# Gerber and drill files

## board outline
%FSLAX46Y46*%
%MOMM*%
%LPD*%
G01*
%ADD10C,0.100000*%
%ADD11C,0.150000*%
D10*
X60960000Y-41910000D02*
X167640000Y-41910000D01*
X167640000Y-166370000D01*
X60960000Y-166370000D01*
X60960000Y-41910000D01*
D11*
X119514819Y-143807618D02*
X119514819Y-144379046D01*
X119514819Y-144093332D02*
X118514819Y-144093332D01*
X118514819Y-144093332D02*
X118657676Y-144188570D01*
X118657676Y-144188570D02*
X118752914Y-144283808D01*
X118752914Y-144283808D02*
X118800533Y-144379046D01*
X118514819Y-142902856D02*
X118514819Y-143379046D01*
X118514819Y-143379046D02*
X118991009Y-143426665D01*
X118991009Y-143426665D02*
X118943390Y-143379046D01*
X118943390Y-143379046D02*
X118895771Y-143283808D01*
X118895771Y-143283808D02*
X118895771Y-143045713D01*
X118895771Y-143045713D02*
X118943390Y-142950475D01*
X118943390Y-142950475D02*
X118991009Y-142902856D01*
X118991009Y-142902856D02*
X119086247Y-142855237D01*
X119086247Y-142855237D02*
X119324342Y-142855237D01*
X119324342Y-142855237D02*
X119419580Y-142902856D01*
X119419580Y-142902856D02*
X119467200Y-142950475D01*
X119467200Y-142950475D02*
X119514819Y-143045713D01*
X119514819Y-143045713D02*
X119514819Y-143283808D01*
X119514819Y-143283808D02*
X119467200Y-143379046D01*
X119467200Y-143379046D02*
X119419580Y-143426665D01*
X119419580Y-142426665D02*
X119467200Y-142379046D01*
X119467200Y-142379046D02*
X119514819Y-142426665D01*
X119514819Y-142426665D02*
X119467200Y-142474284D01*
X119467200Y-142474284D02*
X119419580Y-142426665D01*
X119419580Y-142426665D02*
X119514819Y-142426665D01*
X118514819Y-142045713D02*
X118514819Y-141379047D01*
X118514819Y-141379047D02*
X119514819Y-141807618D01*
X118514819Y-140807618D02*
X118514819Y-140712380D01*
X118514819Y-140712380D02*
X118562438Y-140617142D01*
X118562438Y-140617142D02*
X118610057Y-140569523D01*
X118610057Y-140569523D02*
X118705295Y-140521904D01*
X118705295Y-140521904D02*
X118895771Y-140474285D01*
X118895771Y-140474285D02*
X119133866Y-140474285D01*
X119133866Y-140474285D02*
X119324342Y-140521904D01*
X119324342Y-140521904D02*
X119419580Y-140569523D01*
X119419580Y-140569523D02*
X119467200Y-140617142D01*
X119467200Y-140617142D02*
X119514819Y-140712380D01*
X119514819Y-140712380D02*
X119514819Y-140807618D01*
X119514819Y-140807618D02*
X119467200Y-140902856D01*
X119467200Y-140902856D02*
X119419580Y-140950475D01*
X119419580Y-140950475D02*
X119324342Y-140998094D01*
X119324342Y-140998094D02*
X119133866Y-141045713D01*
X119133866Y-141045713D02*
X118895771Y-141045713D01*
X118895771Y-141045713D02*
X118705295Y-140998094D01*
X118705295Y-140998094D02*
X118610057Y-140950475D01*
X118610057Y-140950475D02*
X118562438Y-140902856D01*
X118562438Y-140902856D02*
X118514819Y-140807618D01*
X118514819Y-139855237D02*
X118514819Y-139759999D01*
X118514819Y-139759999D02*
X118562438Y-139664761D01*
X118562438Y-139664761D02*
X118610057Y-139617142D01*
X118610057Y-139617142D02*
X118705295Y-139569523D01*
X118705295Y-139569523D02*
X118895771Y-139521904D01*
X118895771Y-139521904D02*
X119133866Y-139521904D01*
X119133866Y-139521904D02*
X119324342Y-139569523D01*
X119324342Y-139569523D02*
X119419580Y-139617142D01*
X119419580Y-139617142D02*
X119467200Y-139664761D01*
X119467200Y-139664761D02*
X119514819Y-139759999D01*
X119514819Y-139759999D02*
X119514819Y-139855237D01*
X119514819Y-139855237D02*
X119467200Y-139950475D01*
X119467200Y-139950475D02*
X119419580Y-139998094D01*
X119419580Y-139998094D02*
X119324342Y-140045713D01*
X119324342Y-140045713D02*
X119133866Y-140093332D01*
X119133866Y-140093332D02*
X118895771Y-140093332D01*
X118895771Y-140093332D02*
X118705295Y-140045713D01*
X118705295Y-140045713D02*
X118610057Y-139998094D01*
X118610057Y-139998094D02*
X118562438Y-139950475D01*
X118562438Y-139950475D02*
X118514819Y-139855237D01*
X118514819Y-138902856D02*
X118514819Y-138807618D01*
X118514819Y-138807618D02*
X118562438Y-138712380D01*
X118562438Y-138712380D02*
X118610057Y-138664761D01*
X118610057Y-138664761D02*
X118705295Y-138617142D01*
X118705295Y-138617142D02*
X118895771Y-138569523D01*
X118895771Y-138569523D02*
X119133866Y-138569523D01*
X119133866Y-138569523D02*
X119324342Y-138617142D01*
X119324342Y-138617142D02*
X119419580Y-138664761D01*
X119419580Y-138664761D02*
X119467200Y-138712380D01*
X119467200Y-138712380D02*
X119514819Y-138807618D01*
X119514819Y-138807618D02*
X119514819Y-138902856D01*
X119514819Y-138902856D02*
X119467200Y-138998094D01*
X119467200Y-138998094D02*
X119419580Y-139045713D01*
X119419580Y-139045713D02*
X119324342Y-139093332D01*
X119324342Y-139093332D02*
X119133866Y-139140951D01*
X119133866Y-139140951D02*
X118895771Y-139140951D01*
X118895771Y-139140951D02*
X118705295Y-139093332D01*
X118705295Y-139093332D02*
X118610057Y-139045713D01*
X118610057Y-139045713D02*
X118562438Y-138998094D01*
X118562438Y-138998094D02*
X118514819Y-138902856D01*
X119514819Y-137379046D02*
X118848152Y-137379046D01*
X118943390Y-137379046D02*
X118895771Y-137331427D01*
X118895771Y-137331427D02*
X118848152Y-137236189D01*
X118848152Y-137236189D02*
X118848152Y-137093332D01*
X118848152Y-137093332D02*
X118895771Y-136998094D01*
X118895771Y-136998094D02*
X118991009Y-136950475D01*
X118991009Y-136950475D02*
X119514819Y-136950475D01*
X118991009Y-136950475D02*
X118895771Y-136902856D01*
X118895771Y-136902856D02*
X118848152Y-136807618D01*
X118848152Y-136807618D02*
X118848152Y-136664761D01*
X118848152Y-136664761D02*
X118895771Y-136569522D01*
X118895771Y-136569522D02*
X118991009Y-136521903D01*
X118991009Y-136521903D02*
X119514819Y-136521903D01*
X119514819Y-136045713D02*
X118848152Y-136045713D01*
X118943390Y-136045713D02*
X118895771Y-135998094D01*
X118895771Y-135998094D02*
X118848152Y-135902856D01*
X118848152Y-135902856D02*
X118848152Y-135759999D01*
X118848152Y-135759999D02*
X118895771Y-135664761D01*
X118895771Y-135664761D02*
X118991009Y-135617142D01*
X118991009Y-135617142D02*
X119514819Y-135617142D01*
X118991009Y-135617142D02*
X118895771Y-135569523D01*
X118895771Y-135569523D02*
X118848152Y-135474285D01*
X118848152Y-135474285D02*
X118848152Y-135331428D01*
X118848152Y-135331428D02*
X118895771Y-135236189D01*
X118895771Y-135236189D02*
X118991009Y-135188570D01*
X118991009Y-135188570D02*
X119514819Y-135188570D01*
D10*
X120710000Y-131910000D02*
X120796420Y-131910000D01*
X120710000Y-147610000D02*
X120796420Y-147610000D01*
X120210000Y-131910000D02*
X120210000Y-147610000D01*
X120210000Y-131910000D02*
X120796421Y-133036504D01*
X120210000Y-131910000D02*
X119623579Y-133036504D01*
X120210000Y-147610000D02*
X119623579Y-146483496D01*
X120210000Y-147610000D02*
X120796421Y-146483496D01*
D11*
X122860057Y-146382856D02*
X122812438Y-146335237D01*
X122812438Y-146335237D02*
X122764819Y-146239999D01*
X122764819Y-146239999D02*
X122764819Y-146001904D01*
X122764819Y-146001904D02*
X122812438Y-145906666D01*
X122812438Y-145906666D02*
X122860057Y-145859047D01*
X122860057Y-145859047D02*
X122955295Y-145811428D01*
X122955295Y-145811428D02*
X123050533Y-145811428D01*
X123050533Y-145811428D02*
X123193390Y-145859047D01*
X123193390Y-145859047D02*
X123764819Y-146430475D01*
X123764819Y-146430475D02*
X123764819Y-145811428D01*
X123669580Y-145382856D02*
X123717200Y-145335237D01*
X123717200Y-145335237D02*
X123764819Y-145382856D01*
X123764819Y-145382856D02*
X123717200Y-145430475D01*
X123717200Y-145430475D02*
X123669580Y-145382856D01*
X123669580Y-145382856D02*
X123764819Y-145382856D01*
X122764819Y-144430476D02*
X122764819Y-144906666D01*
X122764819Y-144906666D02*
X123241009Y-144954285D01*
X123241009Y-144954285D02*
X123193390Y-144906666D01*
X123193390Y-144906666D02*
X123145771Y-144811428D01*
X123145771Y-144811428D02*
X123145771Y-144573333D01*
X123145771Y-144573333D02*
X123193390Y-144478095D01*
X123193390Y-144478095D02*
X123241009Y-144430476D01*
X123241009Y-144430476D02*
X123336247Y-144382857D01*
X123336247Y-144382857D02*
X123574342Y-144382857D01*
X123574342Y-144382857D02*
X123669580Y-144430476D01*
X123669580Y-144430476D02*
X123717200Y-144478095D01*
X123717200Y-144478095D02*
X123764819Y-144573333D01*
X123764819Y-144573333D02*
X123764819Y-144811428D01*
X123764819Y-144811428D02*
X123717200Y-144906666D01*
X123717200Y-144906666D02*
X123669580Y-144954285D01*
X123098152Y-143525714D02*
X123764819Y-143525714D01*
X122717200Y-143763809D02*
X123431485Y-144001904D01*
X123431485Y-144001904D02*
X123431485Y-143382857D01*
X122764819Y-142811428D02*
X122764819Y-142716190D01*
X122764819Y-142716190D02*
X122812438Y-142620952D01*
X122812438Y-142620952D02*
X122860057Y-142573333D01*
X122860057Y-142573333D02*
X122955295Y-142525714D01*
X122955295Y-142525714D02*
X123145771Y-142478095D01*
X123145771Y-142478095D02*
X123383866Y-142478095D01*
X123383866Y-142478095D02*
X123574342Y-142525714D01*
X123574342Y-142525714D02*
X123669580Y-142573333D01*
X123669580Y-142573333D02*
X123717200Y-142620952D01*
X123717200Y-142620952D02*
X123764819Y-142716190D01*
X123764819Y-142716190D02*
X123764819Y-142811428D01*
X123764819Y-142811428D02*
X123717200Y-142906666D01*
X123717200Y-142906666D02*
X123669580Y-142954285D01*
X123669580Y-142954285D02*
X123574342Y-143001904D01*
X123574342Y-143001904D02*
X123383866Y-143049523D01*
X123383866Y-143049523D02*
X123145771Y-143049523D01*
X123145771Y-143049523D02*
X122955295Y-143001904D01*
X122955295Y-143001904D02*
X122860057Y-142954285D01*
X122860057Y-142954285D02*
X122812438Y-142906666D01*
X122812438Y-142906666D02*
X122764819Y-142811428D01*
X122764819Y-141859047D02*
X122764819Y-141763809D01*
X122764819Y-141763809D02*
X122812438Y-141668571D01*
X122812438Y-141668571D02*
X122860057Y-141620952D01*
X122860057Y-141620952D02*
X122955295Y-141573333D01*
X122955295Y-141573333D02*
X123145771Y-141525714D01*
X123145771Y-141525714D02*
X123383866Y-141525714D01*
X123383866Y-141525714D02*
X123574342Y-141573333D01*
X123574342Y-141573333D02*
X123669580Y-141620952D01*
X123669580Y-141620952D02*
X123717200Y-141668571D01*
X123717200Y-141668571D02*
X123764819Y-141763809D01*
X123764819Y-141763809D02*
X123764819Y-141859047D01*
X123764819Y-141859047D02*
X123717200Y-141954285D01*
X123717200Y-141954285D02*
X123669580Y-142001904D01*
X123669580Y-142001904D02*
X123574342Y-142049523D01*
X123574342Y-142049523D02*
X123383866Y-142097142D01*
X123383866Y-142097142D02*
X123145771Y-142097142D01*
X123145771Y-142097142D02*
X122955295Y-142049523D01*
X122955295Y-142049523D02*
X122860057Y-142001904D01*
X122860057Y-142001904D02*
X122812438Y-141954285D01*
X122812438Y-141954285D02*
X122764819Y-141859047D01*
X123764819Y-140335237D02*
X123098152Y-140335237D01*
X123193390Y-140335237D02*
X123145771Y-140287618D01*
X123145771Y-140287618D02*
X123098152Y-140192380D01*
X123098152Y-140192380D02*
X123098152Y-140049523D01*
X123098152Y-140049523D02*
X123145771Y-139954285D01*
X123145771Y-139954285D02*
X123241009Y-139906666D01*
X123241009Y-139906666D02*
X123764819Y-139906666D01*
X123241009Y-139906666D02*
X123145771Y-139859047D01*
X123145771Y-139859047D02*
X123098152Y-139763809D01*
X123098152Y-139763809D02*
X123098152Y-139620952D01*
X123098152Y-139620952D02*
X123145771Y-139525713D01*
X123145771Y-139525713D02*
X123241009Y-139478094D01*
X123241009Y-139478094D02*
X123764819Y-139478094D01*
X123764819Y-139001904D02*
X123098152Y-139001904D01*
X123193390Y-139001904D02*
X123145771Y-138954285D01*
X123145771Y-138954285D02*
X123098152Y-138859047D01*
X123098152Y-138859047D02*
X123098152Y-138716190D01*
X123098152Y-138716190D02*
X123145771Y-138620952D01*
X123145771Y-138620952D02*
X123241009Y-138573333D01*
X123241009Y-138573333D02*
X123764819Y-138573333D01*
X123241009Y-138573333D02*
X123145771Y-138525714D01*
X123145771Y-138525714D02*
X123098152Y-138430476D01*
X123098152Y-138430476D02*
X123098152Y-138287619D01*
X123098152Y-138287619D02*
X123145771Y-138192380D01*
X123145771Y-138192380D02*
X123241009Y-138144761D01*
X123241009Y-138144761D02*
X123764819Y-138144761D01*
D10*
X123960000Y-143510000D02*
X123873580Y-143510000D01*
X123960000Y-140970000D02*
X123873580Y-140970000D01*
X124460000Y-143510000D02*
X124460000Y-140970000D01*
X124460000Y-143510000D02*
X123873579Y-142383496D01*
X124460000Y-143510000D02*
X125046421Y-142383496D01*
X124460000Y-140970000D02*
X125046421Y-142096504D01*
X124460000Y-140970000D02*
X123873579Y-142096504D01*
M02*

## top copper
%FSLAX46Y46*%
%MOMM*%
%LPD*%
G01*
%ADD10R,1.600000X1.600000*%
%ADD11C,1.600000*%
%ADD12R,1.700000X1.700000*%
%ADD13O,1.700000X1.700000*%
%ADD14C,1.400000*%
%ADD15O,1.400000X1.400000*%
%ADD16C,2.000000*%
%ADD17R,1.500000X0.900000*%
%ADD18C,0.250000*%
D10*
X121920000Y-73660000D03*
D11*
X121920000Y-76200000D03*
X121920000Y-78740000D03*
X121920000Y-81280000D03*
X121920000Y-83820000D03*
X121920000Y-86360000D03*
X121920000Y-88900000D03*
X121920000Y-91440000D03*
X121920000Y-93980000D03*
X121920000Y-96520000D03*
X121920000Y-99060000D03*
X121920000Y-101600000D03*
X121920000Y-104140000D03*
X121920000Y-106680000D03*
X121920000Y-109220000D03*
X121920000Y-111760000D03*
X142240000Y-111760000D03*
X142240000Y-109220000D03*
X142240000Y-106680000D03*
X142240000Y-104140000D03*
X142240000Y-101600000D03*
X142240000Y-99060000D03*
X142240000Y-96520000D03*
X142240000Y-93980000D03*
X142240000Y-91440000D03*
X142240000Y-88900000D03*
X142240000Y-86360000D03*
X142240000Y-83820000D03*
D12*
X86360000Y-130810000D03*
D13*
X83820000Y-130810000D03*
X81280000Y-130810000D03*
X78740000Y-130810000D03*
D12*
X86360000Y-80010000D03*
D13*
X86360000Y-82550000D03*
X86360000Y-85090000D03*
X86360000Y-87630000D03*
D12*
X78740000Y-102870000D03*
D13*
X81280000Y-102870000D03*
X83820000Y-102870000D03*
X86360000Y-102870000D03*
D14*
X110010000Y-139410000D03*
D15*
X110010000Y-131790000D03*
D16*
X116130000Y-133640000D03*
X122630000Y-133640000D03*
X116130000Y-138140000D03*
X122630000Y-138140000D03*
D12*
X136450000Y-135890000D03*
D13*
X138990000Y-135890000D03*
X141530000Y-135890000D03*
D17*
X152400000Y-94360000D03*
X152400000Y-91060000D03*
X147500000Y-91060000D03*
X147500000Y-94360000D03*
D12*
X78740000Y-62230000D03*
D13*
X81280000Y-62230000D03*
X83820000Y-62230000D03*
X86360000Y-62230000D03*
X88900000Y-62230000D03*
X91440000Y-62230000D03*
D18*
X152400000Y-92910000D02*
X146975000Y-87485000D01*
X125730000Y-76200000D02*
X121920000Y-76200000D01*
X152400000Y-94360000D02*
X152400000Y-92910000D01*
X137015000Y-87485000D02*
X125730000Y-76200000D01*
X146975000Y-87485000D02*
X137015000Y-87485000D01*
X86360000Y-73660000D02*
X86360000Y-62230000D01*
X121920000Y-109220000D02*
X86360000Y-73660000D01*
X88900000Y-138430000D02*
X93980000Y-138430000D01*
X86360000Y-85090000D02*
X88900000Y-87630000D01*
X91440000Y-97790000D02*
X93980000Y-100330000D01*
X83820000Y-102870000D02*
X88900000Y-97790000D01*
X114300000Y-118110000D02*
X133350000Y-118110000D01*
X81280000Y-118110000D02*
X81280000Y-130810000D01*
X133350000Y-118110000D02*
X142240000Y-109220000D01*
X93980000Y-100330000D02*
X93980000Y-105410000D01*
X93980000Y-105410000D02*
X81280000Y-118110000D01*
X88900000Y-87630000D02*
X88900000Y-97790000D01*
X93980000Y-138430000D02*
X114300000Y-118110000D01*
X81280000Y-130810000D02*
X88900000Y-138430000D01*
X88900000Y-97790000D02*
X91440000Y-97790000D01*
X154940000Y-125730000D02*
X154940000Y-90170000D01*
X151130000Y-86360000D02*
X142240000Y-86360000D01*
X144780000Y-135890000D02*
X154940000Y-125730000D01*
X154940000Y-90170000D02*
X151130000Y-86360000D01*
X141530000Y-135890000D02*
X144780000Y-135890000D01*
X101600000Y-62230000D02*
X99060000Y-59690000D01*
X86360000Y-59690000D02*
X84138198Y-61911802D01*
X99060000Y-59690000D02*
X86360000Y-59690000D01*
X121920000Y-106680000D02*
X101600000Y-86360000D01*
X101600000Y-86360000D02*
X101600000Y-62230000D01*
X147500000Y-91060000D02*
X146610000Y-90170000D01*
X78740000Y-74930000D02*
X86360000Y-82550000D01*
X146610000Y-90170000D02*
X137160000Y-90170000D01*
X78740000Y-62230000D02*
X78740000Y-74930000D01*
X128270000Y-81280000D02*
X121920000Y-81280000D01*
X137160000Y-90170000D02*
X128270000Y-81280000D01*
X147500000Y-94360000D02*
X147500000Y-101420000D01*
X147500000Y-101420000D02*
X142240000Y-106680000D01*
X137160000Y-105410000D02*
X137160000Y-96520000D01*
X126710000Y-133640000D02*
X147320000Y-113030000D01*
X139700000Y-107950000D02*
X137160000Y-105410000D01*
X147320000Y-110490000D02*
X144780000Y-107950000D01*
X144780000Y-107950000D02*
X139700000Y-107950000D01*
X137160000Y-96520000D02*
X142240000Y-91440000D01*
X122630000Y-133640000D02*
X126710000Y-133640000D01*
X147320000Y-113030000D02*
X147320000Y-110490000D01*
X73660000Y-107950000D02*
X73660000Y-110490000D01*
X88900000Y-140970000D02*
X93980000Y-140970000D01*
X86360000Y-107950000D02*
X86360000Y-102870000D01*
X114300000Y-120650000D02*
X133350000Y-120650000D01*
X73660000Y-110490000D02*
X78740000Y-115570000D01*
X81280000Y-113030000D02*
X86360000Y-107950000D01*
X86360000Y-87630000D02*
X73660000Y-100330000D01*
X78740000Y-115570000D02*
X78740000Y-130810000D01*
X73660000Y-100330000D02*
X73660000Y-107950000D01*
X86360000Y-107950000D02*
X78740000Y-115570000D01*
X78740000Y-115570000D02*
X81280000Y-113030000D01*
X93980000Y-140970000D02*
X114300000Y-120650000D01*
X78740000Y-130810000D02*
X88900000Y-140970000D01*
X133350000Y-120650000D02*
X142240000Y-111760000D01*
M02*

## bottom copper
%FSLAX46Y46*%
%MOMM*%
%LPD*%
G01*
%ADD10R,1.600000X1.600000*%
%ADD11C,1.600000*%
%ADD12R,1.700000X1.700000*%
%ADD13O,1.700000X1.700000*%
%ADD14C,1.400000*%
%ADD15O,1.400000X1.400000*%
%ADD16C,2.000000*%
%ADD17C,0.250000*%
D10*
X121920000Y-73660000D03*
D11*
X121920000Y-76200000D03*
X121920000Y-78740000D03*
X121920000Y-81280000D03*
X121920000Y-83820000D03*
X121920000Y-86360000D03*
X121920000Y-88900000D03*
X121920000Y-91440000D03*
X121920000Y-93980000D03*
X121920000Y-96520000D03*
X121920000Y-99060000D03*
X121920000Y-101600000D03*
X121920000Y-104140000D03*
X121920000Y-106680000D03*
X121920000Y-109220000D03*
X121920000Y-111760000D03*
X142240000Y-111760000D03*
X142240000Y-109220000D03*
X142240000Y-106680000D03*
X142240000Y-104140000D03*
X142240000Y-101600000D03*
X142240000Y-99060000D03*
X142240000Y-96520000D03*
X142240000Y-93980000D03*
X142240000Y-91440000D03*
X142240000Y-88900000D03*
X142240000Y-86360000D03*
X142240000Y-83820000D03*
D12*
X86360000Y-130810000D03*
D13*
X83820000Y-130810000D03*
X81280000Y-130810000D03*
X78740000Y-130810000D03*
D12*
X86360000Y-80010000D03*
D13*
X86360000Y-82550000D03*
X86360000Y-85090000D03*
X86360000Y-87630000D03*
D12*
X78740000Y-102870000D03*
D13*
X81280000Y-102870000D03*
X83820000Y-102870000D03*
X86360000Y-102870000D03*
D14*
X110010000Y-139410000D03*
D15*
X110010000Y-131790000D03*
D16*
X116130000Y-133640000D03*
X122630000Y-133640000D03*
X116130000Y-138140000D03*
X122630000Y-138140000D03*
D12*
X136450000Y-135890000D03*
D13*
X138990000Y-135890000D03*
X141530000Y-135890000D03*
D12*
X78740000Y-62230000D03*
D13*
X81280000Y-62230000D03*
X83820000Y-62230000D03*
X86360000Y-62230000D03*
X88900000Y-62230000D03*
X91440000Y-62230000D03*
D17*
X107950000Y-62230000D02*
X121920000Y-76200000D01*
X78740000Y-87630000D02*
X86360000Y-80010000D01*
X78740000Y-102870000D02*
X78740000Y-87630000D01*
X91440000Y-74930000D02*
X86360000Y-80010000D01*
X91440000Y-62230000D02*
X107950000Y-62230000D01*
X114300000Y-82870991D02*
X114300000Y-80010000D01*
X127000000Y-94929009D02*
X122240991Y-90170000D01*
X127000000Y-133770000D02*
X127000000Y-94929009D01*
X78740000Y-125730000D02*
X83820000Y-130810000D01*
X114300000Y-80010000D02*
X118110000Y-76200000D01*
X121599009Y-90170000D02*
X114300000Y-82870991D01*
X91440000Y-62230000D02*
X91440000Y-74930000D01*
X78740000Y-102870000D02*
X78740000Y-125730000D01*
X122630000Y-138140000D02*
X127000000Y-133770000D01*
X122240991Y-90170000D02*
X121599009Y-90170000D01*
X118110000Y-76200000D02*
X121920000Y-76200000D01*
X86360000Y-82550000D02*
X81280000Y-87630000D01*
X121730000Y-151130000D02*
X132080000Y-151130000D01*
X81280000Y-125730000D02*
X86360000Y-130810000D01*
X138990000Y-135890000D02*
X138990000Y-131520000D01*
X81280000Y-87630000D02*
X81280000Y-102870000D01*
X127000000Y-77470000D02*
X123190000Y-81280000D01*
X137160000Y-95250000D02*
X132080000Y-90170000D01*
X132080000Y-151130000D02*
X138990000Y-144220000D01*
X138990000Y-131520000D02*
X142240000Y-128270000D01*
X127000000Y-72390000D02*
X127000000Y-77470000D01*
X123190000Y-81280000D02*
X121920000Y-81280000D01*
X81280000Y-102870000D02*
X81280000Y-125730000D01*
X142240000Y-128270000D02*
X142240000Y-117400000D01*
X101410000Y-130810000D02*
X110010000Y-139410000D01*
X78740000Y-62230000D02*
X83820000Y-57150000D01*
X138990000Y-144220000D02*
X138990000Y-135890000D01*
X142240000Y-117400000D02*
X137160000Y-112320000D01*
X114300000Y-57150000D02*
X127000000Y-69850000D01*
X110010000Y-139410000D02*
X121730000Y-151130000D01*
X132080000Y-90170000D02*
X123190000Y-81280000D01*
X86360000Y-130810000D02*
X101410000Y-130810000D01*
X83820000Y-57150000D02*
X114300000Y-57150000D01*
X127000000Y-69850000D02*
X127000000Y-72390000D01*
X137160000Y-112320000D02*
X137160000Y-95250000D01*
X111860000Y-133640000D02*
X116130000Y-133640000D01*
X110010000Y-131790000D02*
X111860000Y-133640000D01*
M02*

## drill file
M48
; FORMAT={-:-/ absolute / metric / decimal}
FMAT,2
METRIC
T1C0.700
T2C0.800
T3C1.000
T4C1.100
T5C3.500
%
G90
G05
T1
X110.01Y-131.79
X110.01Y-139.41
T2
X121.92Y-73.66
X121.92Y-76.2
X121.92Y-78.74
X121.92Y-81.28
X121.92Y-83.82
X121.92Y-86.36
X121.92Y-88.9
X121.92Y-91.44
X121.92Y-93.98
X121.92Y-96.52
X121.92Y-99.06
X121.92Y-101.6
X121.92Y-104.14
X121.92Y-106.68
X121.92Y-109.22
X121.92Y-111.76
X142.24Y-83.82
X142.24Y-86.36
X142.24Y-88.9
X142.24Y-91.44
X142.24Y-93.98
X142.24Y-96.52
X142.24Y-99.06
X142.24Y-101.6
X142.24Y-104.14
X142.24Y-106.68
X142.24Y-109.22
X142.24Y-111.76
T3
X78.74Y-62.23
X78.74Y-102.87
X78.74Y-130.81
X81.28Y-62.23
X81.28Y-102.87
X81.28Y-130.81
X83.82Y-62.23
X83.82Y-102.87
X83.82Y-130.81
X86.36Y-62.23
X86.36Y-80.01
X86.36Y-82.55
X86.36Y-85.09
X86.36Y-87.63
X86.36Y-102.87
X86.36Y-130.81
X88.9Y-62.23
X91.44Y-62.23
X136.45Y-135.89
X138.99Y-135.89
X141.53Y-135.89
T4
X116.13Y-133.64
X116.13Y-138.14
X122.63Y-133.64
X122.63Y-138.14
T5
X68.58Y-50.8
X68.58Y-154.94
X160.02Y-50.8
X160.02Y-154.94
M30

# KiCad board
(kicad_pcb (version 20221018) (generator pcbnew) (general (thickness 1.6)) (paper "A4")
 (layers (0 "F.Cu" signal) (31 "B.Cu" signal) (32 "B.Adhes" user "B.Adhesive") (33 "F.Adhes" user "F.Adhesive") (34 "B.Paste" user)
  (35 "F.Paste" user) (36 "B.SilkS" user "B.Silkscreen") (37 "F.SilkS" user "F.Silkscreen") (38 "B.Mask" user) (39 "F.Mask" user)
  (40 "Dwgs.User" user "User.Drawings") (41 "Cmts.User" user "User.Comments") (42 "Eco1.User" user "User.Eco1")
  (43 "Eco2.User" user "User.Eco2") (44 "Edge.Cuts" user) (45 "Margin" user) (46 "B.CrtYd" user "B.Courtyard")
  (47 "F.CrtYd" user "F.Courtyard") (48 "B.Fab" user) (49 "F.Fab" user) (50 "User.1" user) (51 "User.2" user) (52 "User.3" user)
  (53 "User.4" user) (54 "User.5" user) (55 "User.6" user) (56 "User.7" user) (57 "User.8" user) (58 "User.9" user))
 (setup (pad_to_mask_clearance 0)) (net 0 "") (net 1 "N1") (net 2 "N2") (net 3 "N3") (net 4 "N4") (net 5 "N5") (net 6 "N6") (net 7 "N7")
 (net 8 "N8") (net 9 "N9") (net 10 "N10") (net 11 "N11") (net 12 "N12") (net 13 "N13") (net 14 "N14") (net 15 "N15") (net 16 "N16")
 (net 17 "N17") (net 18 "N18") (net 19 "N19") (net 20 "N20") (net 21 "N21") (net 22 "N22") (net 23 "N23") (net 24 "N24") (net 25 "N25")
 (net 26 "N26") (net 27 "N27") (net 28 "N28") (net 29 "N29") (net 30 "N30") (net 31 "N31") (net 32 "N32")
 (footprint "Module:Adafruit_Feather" (layer "F.Cu") (at 121.92 73.66)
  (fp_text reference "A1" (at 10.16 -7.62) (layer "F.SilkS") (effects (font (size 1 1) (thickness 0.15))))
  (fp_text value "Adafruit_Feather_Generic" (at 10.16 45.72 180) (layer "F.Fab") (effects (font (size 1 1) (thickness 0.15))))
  (pad "1" thru_hole rect (at 0 0 180) (size 1.6 1.6) (drill 0.8) (layers "*.Cu" "*.Mask") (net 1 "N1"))
  (pad "2" thru_hole circle (at 0 2.54 180) (size 1.6 1.6) (drill 0.8) (layers "*.Cu" "*.Mask") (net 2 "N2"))
  (pad "3" thru_hole circle (at 0 5.08 180) (size 1.6 1.6) (drill 0.8) (layers "*.Cu" "*.Mask") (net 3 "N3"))
  (pad "4" thru_hole circle (at 0 7.62 180) (size 1.6 1.6) (drill 0.8) (layers "*.Cu" "*.Mask") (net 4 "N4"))
  (pad "5" thru_hole circle (at 0 10.16 180) (size 1.6 1.6) (drill 0.8) (layers "*.Cu" "*.Mask") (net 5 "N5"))
  (pad "6" thru_hole circle (at 0 12.7 180) (size 1.6 1.6) (drill 0.8) (layers "*.Cu" "*.Mask") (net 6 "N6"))
  (pad "7" thru_hole circle (at 0 15.24 180) (size 1.6 1.6) (drill 0.8) (layers "*.Cu" "*.Mask") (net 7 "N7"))
  (pad "8" thru_hole circle (at 0 17.78 180) (size 1.6 1.6) (drill 0.8) (layers "*.Cu" "*.Mask") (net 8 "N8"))
  (pad "9" thru_hole circle (at 0 20.32 180) (size 1.6 1.6) (drill 0.8) (layers "*.Cu" "*.Mask") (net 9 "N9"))
  (pad "10" thru_hole circle (at 0 22.86 180) (size 1.6 1.6) (drill 0.8) (layers "*.Cu" "*.Mask") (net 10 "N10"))
  (pad "11" thru_hole circle (at 0 25.4 180) (size 1.6 1.6) (drill 0.8) (layers "*.Cu" "*.Mask") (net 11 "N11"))
  (pad "12" thru_hole circle (at 0 27.94 180) (size 1.6 1.6) (drill 0.8) (layers "*.Cu" "*.Mask") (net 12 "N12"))
  (pad "13" thru_hole circle (at 0 30.48 180) (size 1.6 1.6) (drill 0.8) (layers "*.Cu" "*.Mask") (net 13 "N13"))
  (pad "14" thru_hole circle (at 0 33.02 180) (size 1.6 1.6) (drill 0.8) (layers "*.Cu" "*.Mask") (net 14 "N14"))
  (pad "15" thru_hole circle (at 0 35.56 180) (size 1.6 1.6) (drill 0.8) (layers "*.Cu" "*.Mask") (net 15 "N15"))
  (pad "16" thru_hole circle (at 0 38.1 180) (size 1.6 1.6) (drill 0.8) (layers "*.Cu" "*.Mask") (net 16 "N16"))
  (pad "17" thru_hole circle (at 20.32 38.1 180) (size 1.6 1.6) (drill 0.8) (layers "*.Cu" "*.Mask") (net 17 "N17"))
  (pad "18" thru_hole circle (at 20.32 35.56 180) (size 1.6 1.6) (drill 0.8) (layers "*.Cu" "*.Mask") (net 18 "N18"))
  (pad "19" thru_hole circle (at 20.32 33.02 180) (size 1.6 1.6) (drill 0.8) (layers "*.Cu" "*.Mask") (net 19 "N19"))
  (pad "20" thru_hole circle (at 20.32 30.48 180) (size 1.6 1.6) (drill 0.8) (layers "*.Cu" "*.Mask") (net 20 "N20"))
  (pad "21" thru_hole circle (at 20.32 27.94 180) (size 1.6 1.6) (drill 0.8) (layers "*.Cu" "*.Mask") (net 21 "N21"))
  (pad "22" thru_hole circle (at 20.32 25.4 180) (size 1.6 1.6) (drill 0.8) (layers "*.Cu" "*.Mask") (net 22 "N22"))
  (pad "23" thru_hole circle (at 20.32 22.86 180) (size 1.6 1.6) (drill 0.8) (layers "*.Cu" "*.Mask") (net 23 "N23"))
  (pad "24" thru_hole circle (at 20.32 20.32 180) (size 1.6 1.6) (drill 0.8) (layers "*.Cu" "*.Mask") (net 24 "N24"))
  (pad "25" thru_hole circle (at 20.32 17.78 180) (size 1.6 1.6) (drill 0.8) (layers "*.Cu" "*.Mask") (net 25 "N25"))
  (pad "26" thru_hole circle (at 20.32 15.24 180) (size 1.6 1.6) (drill 0.8) (layers "*.Cu" "*.Mask") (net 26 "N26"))
  (pad "27" thru_hole circle (at 20.32 12.7 180) (size 1.6 1.6) (drill 0.8) (layers "*.Cu" "*.Mask") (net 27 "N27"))
  (pad "28" thru_hole circle (at 20.32 10.16 180) (size 1.6 1.6) (drill 0.8) (layers "*.Cu" "*.Mask") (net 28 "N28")))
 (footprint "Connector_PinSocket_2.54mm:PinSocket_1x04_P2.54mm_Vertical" (layer "F.Cu") (at 86.36 130.81 -90)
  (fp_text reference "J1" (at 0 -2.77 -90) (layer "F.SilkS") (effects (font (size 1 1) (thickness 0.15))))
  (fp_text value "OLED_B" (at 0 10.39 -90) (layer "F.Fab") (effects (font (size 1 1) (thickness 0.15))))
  (pad "1" thru_hole rect (at 0 0 270) (size 1.7 1.7) (drill 1) (layers "*.Cu" "*.Mask") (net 4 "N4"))
  (pad "2" thru_hole oval (at 0 2.54 270) (size 1.7 1.7) (drill 1) (layers "*.Cu" "*.Mask") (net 2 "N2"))
  (pad "3" thru_hole oval (at 0 5.08 270) (size 1.7 1.7) (drill 1) (layers "*.Cu" "*.Mask") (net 18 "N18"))
  (pad "4" thru_hole oval (at 0 7.62 270) (size 1.7 1.7) (drill 1) (layers "*.Cu" "*.Mask") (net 17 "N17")))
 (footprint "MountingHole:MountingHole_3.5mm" (layer "F.Cu") (at 68.58 154.94)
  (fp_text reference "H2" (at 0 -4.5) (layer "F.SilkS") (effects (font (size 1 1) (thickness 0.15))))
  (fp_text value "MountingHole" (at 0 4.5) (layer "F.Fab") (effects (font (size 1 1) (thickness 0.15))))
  (pad "" np_thru_hole circle (at 0 0) (size 3.5 3.5) (drill 3.5) (layers "*.Cu" "*.Mask")))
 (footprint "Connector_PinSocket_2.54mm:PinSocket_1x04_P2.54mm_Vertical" (layer "F.Cu") (at 86.36 80.01)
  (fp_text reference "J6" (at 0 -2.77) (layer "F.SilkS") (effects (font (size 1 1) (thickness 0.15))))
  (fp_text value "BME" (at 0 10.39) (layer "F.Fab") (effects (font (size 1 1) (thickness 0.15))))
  (pad "1" thru_hole rect (at 0 0) (size 1.7 1.7) (drill 1) (layers "*.Cu" "*.Mask") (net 2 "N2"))
  (pad "2" thru_hole oval (at 0 2.54) (size 1.7 1.7) (drill 1) (layers "*.Cu" "*.Mask") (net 4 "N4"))
  (pad "3" thru_hole oval (at 0 5.08) (size 1.7 1.7) (drill 1) (layers "*.Cu" "*.Mask") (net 18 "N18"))
  (pad "4" thru_hole oval (at 0 7.62) (size 1.7 1.7) (drill 1) (layers "*.Cu" "*.Mask") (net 17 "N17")))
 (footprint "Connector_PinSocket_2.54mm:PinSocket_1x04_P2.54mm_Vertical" (layer "F.Cu") (at 78.74 102.87 90)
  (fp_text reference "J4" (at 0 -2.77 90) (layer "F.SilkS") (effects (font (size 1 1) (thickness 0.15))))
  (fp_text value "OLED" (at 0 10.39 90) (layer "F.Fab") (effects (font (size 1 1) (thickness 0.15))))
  (pad "1" thru_hole rect (at 0 0 90) (size 1.7 1.7) (drill 1) (layers "*.Cu" "*.Mask") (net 2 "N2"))
  (pad "2" thru_hole oval (at 0 2.54 90) (size 1.7 1.7) (drill 1) (layers "*.Cu" "*.Mask") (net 4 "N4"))
  (pad "3" thru_hole oval (at 0 5.08 90) (size 1.7 1.7) (drill 1) (layers "*.Cu" "*.Mask") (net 18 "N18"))
  (pad "4" thru_hole oval (at 0 7.62 90) (size 1.7 1.7) (drill 1) (layers "*.Cu" "*.Mask") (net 17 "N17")))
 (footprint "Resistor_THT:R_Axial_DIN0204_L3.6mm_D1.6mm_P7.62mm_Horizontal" (layer "F.Cu") (at 110.01 139.41 90)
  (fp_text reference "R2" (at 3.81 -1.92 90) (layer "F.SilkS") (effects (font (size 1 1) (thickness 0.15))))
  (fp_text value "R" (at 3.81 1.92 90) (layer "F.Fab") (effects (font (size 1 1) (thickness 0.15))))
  (pad "1" thru_hole circle (at 0 0 90) (size 1.4 1.4) (drill 0.7) (layers "*.Cu" "*.Mask") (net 4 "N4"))
  (pad "2" thru_hole oval (at 7.62 0 90) (size 1.4 1.4) (drill 0.7) (layers "*.Cu" "*.Mask") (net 25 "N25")))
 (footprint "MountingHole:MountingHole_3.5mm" (layer "F.Cu") (at 68.58 50.8)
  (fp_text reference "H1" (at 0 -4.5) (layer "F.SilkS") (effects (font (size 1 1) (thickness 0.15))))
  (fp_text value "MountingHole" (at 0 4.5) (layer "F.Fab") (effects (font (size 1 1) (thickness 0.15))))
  (pad "" np_thru_hole circle (at 0 0) (size 3.5 3.5) (drill 3.5) (layers "*.Cu" "*.Mask")))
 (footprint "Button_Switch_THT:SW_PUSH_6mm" (layer "F.Cu") (at 116.13 133.64)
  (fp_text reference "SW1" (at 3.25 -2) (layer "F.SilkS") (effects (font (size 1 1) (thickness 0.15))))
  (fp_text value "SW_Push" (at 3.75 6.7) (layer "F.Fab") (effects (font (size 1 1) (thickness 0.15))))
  (pad "1" thru_hole circle (at 0 0 90) (size 2 2) (drill 1.1) (layers "*.Cu" "*.Mask") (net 25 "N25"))
  (pad "1" thru_hole circle (at 6.5 0 90) (size 2 2) (drill 1.1) (layers "*.Cu" "*.Mask") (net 25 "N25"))
  (pad "2" thru_hole circle (at 0 4.5 90) (size 2 2) (drill 1.1) (layers "*.Cu" "*.Mask") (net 2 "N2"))
  (pad "2" thru_hole circle (at 6.5 4.5 90) (size 2 2) (drill 1.1) (layers "*.Cu" "*.Mask") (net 2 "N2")))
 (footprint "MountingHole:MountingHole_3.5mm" (layer "F.Cu") (at 160.02 50.8)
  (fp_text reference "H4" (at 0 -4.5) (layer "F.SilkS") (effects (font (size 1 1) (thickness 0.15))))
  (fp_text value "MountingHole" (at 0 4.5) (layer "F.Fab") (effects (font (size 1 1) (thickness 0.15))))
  (pad "" np_thru_hole circle (at 0 0) (size 3.5 3.5) (drill 3.5) (layers "*.Cu" "*.Mask")))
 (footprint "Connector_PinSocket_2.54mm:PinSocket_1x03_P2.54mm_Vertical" (layer "F.Cu") (at 136.45 135.89 90)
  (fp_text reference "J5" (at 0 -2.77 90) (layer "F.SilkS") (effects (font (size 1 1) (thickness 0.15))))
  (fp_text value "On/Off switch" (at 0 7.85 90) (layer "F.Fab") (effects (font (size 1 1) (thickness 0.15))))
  (pad "1" thru_hole rect (at 0 0 90) (size 1.7 1.7) (drill 1) (layers "*.Cu" "*.Mask") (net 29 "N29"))
  (pad "2" thru_hole oval (at 0 2.54 90) (size 1.7 1.7) (drill 1) (layers "*.Cu" "*.Mask") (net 4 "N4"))
  (pad "3" thru_hole oval (at 0 5.08 90) (size 1.7 1.7) (drill 1) (layers "*.Cu" "*.Mask") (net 27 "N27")))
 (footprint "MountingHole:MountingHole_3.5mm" (layer "F.Cu") (at 160.02 154.94)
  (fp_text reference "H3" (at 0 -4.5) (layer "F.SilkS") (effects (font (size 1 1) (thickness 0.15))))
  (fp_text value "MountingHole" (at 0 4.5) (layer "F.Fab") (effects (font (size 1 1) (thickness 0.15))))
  (pad "" np_thru_hole circle (at 0 0) (size 3.5 3.5) (drill 3.5) (layers "*.Cu" "*.Mask")))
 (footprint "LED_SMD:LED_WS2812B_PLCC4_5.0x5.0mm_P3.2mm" (layer "F.Cu") (at 149.95 92.71 180)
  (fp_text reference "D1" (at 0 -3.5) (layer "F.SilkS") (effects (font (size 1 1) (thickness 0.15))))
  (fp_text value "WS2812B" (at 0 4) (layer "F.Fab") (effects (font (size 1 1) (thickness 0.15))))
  (pad "1" smd rect (at -2.45 -1.65 180) (size 1.5 0.9) (layers "F.Cu" "F.Paste" "F.Mask") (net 2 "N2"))
  (pad "2" smd rect (at -2.45 1.65 180) (size 1.5 0.9) (layers "F.Cu" "F.Paste" "F.Mask") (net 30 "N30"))
  (pad "3" smd rect (at 2.45 1.65 180) (size 1.5 0.9) (layers "F.Cu" "F.Paste" "F.Mask") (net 4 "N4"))
  (pad "4" smd rect (at 2.45 -1.65 180) (size 1.5 0.9) (layers "F.Cu" "F.Paste" "F.Mask") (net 19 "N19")))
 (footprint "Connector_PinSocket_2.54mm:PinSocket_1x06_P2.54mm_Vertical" (layer "B.Cu") (at 78.74 62.23 -90)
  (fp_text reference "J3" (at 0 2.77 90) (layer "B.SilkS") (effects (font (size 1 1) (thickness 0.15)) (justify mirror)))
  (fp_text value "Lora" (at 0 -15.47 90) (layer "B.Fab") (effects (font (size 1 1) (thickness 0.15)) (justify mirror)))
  (pad "1" thru_hole rect (at 0 0 270) (size 1.7 1.7) (drill 1) (layers "*.Cu" "*.Mask") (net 4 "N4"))
  (pad "2" thru_hole oval (at 0 -2.54 270) (size 1.7 1.7) (drill 1) (layers "*.Cu" "*.Mask") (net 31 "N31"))
  (pad "3" thru_hole oval (at 0 -5.08 270) (size 1.7 1.7) (drill 1) (layers "*.Cu" "*.Mask") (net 14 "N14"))
  (pad "4" thru_hole oval (at 0 -7.62 270) (size 1.7 1.7) (drill 1) (layers "*.Cu" "*.Mask") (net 15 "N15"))
  (pad "5" thru_hole oval (at 0 -10.16 270) (size 1.7 1.7) (drill 1) (layers "*.Cu" "*.Mask") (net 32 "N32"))
  (pad "6" thru_hole oval (at 0 -12.7 270) (size 1.7 1.7) (drill 1) (layers "*.Cu" "*.Mask") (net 2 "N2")))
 (gr_rect (start 60.96 41.91) (end 167.64 166.37) (stroke (width 0.1) (type default)) (fill none) (layer "Edge.Cuts"))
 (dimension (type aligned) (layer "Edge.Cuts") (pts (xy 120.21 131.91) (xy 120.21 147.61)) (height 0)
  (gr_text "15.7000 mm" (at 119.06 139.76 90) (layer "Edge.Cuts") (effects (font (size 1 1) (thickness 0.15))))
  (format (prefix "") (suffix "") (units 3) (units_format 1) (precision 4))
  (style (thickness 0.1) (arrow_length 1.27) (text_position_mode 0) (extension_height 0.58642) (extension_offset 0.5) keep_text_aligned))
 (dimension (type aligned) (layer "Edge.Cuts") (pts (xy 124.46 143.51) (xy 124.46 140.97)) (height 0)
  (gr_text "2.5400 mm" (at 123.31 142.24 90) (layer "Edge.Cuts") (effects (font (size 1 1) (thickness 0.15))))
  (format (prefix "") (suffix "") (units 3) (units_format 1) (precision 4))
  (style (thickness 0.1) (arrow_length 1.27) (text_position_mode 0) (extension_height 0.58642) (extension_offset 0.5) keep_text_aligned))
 (segment (start 152.4 92.91) (end 146.975 87.485) (width 0.25) (layer "F.Cu") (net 2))
 (segment (start 125.73 76.2) (end 121.92 76.2) (width 0.25) (layer "F.Cu") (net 2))
 (segment (start 152.4 94.36) (end 152.4 92.91) (width 0.25) (layer "F.Cu") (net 2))
 (segment (start 137.015 87.485) (end 125.73 76.2) (width 0.25) (layer "F.Cu") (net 2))
 (segment (start 146.975 87.485) (end 137.015 87.485) (width 0.25) (layer "F.Cu") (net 2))
 (segment (start 107.95 62.23) (end 121.92 76.2) (width 0.25) (layer "B.Cu") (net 2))
 (segment (start 78.74 87.63) (end 86.36 80.01) (width 0.25) (layer "B.Cu") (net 2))
 (segment (start 78.74 102.87) (end 78.74 87.63) (width 0.25) (layer "B.Cu") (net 2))
 (segment (start 91.44 74.93) (end 86.36 80.01) (width 0.25) (layer "B.Cu") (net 2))
 (segment (start 91.44 62.23) (end 107.95 62.23) (width 0.25) (layer "B.Cu") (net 2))
 (segment (start 114.3 82.870991) (end 114.3 80.01) (width 0.25) (layer "B.Cu") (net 2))
 (segment (start 127 94.929009) (end 122.240991 90.17) (width 0.25) (layer "B.Cu") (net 2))
 (segment (start 127 133.77) (end 127 94.929009) (width 0.25) (layer "B.Cu") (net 2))
 (segment (start 78.74 125.73) (end 83.82 130.81) (width 0.25) (layer "B.Cu") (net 2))
 (segment (start 114.3 80.01) (end 118.11 76.2) (width 0.25) (layer "B.Cu") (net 2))
 (segment (start 121.599009 90.17) (end 114.3 82.870991) (width 0.25) (layer "B.Cu") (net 2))
 (segment (start 91.44 62.23) (end 91.44 74.93) (width 0.25) (layer "B.Cu") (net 2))
 (segment (start 78.74 102.87) (end 78.74 125.73) (width 0.25) (layer "B.Cu") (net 2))
 (segment (start 122.63 138.14) (end 127 133.77) (width 0.25) (layer "B.Cu") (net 2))
 (segment (start 122.240991 90.17) (end 121.599009 90.17) (width 0.25) (layer "B.Cu") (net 2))
 (segment (start 118.11 76.2) (end 121.92 76.2) (width 0.25) (layer "B.Cu") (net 2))
 (segment (start 86.36 73.66) (end 86.36 62.23) (width 0.25) (layer "F.Cu") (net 15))
 (segment (start 121.92 109.22) (end 86.36 73.66) (width 0.25) (layer "F.Cu") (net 15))
 (segment (start 88.9 138.43) (end 93.98 138.43) (width 0.25) (layer "F.Cu") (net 18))
 (segment (start 86.36 85.09) (end 88.9 87.63) (width 0.25) (layer "F.Cu") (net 18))
 (segment (start 91.44 97.79) (end 93.98 100.33) (width 0.25) (layer "F.Cu") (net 18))
 (segment (start 83.82 102.87) (end 88.9 97.79) (width 0.25) (layer "F.Cu") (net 18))
 (segment (start 114.3 118.11) (end 133.35 118.11) (width 0.25) (layer "F.Cu") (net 18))
 (segment (start 81.28 118.11) (end 81.28 130.81) (width 0.25) (layer "F.Cu") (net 18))
 (segment (start 133.35 118.11) (end 142.24 109.22) (width 0.25) (layer "F.Cu") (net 18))
 (segment (start 93.98 100.33) (end 93.98 105.41) (width 0.25) (layer "F.Cu") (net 18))
 (segment (start 93.98 105.41) (end 81.28 118.11) (width 0.25) (layer "F.Cu") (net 18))
 (segment (start 88.9 87.63) (end 88.9 97.79) (width 0.25) (layer "F.Cu") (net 18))
 (segment (start 93.98 138.43) (end 114.3 118.11) (width 0.25) (layer "F.Cu") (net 18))
 (segment (start 81.28 130.81) (end 88.9 138.43) (width 0.25) (layer "F.Cu") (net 18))
 (segment (start 88.9 97.79) (end 91.44 97.79) (width 0.25) (layer "F.Cu") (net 18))
 (segment (start 154.94 125.73) (end 154.94 90.17) (width 0.25) (layer "F.Cu") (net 27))
 (segment (start 151.13 86.36) (end 142.24 86.36) (width 0.25) (layer "F.Cu") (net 27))
 (segment (start 144.78 135.89) (end 154.94 125.73) (width 0.25) (layer "F.Cu") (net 27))
 (segment (start 154.94 90.17) (end 151.13 86.36) (width 0.25) (layer "F.Cu") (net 27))
 (segment (start 141.53 135.89) (end 144.78 135.89) (width 0.25) (layer "F.Cu") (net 27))
 (segment (start 101.6 62.23) (end 99.06 59.69) (width 0.25) (layer "F.Cu") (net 14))
 (segment (start 86.36 59.69) (end 84.138198 61.911802) (width 0.25) (layer "F.Cu") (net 14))
 (segment (start 99.06 59.69) (end 86.36 59.69) (width 0.25) (layer "F.Cu") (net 14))
 (segment (start 121.92 106.68) (end 101.6 86.36) (width 0.25) (layer "F.Cu") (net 14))
 (segment (start 101.6 86.36) (end 101.6 62.23) (width 0.25) (layer "F.Cu") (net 14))
 (segment (start 147.5 91.06) (end 146.61 90.17) (width 0.25) (layer "F.Cu") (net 4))
 (segment (start 78.74 74.93) (end 86.36 82.55) (width 0.25) (layer "F.Cu") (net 4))
 (segment (start 146.61 90.17) (end 137.16 90.17) (width 0.25) (layer "F.Cu") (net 4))
 (segment (start 78.74 62.23) (end 78.74 74.93) (width 0.25) (layer "F.Cu") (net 4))
 (segment (start 128.27 81.28) (end 121.92 81.28) (width 0.25) (layer "F.Cu") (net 4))
 (segment (start 137.16 90.17) (end 128.27 81.28) (width 0.25) (layer "F.Cu") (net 4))
 (segment (start 86.36 82.55) (end 81.28 87.63) (width 0.25) (layer "B.Cu") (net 4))
 (segment (start 121.73 151.13) (end 132.08 151.13) (width 0.25) (layer "B.Cu") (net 4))
 (segment (start 81.28 125.73) (end 86.36 130.81) (width 0.25) (layer "B.Cu") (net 4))
 (segment (start 138.99 135.89) (end 138.99 131.52) (width 0.25) (layer "B.Cu") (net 4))
 (segment (start 81.28 87.63) (end 81.28 102.87) (width 0.25) (layer "B.Cu") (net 4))
 (segment (start 127 77.47) (end 123.19 81.28) (width 0.25) (layer "B.Cu") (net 4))
 (segment (start 137.16 95.25) (end 132.08 90.17) (width 0.25) (layer "B.Cu") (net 4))
 (segment (start 132.08 151.13) (end 138.99 144.22) (width 0.25) (layer "B.Cu") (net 4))
 (segment (start 138.99 131.52) (end 142.24 128.27) (width 0.25) (layer "B.Cu") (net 4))
 (segment (start 127 72.39) (end 127 77.47) (width 0.25) (layer "B.Cu") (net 4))
 (segment (start 123.19 81.28) (end 121.92 81.28) (width 0.25) (layer "B.Cu") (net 4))
 (segment (start 81.28 102.87) (end 81.28 125.73) (width 0.25) (layer "B.Cu") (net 4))
 (segment (start 142.24 128.27) (end 142.24 117.4) (width 0.25) (layer "B.Cu") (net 4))
 (segment (start 101.41 130.81) (end 110.01 139.41) (width 0.25) (layer "B.Cu") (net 4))
 (segment (start 78.74 62.23) (end 83.82 57.15) (width 0.25) (layer "B.Cu") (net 4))
 (segment (start 138.99 144.22) (end 138.99 135.89) (width 0.25) (layer "B.Cu") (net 4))
 (segment (start 142.24 117.4) (end 137.16 112.32) (width 0.25) (layer "B.Cu") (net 4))
 (segment (start 114.3 57.15) (end 127 69.85) (width 0.25) (layer "B.Cu") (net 4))
 (segment (start 110.01 139.41) (end 121.73 151.13) (width 0.25) (layer "B.Cu") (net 4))
 (segment (start 132.08 90.17) (end 123.19 81.28) (width 0.25) (layer "B.Cu") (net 4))
 (segment (start 86.36 130.81) (end 101.41 130.81) (width 0.25) (layer "B.Cu") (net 4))
 (segment (start 83.82 57.15) (end 114.3 57.15) (width 0.25) (layer "B.Cu") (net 4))
 (segment (start 127 69.85) (end 127 72.39) (width 0.25) (layer "B.Cu") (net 4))
 (segment (start 137.16 112.32) (end 137.16 95.25) (width 0.25) (layer "B.Cu") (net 4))
 (segment (start 147.5 94.36) (end 147.5 101.42) (width 0.25) (layer "F.Cu") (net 19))
 (segment (start 147.5 101.42) (end 142.24 106.68) (width 0.25) (layer "F.Cu") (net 19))
 (segment (start 137.16 105.41) (end 137.16 96.52) (width 0.25) (layer "F.Cu") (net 25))
 (segment (start 126.71 133.64) (end 147.32 113.03) (width 0.25) (layer "F.Cu") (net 25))
 (segment (start 139.7 107.95) (end 137.16 105.41) (width 0.25) (layer "F.Cu") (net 25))
 (segment (start 147.32 110.49) (end 144.78 107.95) (width 0.25) (layer "F.Cu") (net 25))
 (segment (start 144.78 107.95) (end 139.7 107.95) (width 0.25) (layer "F.Cu") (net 25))
 (segment (start 137.16 96.52) (end 142.24 91.44) (width 0.25) (layer "F.Cu") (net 25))
 (segment (start 122.63 133.64) (end 126.71 133.64) (width 0.25) (layer "F.Cu") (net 25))
 (segment (start 147.32 113.03) (end 147.32 110.49) (width 0.25) (layer "F.Cu") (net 25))
 (segment (start 111.86 133.64) (end 116.13 133.64) (width 0.25) (layer "B.Cu") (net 25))
 (segment (start 110.01 131.79) (end 111.86 133.64) (width 0.25) (layer "B.Cu") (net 25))
 (segment (start 73.66 107.95) (end 73.66 110.49) (width 0.25) (layer "F.Cu") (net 17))
 (segment (start 88.9 140.97) (end 93.98 140.97) (width 0.25) (layer "F.Cu") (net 17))
 (segment (start 86.36 107.95) (end 86.36 102.87) (width 0.25) (layer "F.Cu") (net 17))
 (segment (start 114.3 120.65) (end 133.35 120.65) (width 0.25) (layer "F.Cu") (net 17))
 (segment (start 73.66 110.49) (end 78.74 115.57) (width 0.25) (layer "F.Cu") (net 17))
 (segment (start 81.28 113.03) (end 86.36 107.95) (width 0.25) (layer "F.Cu") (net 17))
 (segment (start 86.36 87.63) (end 73.66 100.33) (width 0.25) (layer "F.Cu") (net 17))
 (segment (start 78.74 115.57) (end 78.74 130.81) (width 0.25) (layer "F.Cu") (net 17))
 (segment (start 73.66 100.33) (end 73.66 107.95) (width 0.25) (layer "F.Cu") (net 17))
 (segment (start 86.36 107.95) (end 78.74 115.57) (width 0.25) (layer "F.Cu") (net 17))
 (segment (start 78.74 115.57) (end 81.28 113.03) (width 0.25) (layer "F.Cu") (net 17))
 (segment (start 93.98 140.97) (end 114.3 120.65) (width 0.25) (layer "F.Cu") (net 17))
 (segment (start 78.74 130.81) (end 88.9 140.97) (width 0.25) (layer "F.Cu") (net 17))
 (segment (start 133.35 120.65) (end 142.24 111.76) (width 0.25) (layer "F.Cu") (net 17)))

